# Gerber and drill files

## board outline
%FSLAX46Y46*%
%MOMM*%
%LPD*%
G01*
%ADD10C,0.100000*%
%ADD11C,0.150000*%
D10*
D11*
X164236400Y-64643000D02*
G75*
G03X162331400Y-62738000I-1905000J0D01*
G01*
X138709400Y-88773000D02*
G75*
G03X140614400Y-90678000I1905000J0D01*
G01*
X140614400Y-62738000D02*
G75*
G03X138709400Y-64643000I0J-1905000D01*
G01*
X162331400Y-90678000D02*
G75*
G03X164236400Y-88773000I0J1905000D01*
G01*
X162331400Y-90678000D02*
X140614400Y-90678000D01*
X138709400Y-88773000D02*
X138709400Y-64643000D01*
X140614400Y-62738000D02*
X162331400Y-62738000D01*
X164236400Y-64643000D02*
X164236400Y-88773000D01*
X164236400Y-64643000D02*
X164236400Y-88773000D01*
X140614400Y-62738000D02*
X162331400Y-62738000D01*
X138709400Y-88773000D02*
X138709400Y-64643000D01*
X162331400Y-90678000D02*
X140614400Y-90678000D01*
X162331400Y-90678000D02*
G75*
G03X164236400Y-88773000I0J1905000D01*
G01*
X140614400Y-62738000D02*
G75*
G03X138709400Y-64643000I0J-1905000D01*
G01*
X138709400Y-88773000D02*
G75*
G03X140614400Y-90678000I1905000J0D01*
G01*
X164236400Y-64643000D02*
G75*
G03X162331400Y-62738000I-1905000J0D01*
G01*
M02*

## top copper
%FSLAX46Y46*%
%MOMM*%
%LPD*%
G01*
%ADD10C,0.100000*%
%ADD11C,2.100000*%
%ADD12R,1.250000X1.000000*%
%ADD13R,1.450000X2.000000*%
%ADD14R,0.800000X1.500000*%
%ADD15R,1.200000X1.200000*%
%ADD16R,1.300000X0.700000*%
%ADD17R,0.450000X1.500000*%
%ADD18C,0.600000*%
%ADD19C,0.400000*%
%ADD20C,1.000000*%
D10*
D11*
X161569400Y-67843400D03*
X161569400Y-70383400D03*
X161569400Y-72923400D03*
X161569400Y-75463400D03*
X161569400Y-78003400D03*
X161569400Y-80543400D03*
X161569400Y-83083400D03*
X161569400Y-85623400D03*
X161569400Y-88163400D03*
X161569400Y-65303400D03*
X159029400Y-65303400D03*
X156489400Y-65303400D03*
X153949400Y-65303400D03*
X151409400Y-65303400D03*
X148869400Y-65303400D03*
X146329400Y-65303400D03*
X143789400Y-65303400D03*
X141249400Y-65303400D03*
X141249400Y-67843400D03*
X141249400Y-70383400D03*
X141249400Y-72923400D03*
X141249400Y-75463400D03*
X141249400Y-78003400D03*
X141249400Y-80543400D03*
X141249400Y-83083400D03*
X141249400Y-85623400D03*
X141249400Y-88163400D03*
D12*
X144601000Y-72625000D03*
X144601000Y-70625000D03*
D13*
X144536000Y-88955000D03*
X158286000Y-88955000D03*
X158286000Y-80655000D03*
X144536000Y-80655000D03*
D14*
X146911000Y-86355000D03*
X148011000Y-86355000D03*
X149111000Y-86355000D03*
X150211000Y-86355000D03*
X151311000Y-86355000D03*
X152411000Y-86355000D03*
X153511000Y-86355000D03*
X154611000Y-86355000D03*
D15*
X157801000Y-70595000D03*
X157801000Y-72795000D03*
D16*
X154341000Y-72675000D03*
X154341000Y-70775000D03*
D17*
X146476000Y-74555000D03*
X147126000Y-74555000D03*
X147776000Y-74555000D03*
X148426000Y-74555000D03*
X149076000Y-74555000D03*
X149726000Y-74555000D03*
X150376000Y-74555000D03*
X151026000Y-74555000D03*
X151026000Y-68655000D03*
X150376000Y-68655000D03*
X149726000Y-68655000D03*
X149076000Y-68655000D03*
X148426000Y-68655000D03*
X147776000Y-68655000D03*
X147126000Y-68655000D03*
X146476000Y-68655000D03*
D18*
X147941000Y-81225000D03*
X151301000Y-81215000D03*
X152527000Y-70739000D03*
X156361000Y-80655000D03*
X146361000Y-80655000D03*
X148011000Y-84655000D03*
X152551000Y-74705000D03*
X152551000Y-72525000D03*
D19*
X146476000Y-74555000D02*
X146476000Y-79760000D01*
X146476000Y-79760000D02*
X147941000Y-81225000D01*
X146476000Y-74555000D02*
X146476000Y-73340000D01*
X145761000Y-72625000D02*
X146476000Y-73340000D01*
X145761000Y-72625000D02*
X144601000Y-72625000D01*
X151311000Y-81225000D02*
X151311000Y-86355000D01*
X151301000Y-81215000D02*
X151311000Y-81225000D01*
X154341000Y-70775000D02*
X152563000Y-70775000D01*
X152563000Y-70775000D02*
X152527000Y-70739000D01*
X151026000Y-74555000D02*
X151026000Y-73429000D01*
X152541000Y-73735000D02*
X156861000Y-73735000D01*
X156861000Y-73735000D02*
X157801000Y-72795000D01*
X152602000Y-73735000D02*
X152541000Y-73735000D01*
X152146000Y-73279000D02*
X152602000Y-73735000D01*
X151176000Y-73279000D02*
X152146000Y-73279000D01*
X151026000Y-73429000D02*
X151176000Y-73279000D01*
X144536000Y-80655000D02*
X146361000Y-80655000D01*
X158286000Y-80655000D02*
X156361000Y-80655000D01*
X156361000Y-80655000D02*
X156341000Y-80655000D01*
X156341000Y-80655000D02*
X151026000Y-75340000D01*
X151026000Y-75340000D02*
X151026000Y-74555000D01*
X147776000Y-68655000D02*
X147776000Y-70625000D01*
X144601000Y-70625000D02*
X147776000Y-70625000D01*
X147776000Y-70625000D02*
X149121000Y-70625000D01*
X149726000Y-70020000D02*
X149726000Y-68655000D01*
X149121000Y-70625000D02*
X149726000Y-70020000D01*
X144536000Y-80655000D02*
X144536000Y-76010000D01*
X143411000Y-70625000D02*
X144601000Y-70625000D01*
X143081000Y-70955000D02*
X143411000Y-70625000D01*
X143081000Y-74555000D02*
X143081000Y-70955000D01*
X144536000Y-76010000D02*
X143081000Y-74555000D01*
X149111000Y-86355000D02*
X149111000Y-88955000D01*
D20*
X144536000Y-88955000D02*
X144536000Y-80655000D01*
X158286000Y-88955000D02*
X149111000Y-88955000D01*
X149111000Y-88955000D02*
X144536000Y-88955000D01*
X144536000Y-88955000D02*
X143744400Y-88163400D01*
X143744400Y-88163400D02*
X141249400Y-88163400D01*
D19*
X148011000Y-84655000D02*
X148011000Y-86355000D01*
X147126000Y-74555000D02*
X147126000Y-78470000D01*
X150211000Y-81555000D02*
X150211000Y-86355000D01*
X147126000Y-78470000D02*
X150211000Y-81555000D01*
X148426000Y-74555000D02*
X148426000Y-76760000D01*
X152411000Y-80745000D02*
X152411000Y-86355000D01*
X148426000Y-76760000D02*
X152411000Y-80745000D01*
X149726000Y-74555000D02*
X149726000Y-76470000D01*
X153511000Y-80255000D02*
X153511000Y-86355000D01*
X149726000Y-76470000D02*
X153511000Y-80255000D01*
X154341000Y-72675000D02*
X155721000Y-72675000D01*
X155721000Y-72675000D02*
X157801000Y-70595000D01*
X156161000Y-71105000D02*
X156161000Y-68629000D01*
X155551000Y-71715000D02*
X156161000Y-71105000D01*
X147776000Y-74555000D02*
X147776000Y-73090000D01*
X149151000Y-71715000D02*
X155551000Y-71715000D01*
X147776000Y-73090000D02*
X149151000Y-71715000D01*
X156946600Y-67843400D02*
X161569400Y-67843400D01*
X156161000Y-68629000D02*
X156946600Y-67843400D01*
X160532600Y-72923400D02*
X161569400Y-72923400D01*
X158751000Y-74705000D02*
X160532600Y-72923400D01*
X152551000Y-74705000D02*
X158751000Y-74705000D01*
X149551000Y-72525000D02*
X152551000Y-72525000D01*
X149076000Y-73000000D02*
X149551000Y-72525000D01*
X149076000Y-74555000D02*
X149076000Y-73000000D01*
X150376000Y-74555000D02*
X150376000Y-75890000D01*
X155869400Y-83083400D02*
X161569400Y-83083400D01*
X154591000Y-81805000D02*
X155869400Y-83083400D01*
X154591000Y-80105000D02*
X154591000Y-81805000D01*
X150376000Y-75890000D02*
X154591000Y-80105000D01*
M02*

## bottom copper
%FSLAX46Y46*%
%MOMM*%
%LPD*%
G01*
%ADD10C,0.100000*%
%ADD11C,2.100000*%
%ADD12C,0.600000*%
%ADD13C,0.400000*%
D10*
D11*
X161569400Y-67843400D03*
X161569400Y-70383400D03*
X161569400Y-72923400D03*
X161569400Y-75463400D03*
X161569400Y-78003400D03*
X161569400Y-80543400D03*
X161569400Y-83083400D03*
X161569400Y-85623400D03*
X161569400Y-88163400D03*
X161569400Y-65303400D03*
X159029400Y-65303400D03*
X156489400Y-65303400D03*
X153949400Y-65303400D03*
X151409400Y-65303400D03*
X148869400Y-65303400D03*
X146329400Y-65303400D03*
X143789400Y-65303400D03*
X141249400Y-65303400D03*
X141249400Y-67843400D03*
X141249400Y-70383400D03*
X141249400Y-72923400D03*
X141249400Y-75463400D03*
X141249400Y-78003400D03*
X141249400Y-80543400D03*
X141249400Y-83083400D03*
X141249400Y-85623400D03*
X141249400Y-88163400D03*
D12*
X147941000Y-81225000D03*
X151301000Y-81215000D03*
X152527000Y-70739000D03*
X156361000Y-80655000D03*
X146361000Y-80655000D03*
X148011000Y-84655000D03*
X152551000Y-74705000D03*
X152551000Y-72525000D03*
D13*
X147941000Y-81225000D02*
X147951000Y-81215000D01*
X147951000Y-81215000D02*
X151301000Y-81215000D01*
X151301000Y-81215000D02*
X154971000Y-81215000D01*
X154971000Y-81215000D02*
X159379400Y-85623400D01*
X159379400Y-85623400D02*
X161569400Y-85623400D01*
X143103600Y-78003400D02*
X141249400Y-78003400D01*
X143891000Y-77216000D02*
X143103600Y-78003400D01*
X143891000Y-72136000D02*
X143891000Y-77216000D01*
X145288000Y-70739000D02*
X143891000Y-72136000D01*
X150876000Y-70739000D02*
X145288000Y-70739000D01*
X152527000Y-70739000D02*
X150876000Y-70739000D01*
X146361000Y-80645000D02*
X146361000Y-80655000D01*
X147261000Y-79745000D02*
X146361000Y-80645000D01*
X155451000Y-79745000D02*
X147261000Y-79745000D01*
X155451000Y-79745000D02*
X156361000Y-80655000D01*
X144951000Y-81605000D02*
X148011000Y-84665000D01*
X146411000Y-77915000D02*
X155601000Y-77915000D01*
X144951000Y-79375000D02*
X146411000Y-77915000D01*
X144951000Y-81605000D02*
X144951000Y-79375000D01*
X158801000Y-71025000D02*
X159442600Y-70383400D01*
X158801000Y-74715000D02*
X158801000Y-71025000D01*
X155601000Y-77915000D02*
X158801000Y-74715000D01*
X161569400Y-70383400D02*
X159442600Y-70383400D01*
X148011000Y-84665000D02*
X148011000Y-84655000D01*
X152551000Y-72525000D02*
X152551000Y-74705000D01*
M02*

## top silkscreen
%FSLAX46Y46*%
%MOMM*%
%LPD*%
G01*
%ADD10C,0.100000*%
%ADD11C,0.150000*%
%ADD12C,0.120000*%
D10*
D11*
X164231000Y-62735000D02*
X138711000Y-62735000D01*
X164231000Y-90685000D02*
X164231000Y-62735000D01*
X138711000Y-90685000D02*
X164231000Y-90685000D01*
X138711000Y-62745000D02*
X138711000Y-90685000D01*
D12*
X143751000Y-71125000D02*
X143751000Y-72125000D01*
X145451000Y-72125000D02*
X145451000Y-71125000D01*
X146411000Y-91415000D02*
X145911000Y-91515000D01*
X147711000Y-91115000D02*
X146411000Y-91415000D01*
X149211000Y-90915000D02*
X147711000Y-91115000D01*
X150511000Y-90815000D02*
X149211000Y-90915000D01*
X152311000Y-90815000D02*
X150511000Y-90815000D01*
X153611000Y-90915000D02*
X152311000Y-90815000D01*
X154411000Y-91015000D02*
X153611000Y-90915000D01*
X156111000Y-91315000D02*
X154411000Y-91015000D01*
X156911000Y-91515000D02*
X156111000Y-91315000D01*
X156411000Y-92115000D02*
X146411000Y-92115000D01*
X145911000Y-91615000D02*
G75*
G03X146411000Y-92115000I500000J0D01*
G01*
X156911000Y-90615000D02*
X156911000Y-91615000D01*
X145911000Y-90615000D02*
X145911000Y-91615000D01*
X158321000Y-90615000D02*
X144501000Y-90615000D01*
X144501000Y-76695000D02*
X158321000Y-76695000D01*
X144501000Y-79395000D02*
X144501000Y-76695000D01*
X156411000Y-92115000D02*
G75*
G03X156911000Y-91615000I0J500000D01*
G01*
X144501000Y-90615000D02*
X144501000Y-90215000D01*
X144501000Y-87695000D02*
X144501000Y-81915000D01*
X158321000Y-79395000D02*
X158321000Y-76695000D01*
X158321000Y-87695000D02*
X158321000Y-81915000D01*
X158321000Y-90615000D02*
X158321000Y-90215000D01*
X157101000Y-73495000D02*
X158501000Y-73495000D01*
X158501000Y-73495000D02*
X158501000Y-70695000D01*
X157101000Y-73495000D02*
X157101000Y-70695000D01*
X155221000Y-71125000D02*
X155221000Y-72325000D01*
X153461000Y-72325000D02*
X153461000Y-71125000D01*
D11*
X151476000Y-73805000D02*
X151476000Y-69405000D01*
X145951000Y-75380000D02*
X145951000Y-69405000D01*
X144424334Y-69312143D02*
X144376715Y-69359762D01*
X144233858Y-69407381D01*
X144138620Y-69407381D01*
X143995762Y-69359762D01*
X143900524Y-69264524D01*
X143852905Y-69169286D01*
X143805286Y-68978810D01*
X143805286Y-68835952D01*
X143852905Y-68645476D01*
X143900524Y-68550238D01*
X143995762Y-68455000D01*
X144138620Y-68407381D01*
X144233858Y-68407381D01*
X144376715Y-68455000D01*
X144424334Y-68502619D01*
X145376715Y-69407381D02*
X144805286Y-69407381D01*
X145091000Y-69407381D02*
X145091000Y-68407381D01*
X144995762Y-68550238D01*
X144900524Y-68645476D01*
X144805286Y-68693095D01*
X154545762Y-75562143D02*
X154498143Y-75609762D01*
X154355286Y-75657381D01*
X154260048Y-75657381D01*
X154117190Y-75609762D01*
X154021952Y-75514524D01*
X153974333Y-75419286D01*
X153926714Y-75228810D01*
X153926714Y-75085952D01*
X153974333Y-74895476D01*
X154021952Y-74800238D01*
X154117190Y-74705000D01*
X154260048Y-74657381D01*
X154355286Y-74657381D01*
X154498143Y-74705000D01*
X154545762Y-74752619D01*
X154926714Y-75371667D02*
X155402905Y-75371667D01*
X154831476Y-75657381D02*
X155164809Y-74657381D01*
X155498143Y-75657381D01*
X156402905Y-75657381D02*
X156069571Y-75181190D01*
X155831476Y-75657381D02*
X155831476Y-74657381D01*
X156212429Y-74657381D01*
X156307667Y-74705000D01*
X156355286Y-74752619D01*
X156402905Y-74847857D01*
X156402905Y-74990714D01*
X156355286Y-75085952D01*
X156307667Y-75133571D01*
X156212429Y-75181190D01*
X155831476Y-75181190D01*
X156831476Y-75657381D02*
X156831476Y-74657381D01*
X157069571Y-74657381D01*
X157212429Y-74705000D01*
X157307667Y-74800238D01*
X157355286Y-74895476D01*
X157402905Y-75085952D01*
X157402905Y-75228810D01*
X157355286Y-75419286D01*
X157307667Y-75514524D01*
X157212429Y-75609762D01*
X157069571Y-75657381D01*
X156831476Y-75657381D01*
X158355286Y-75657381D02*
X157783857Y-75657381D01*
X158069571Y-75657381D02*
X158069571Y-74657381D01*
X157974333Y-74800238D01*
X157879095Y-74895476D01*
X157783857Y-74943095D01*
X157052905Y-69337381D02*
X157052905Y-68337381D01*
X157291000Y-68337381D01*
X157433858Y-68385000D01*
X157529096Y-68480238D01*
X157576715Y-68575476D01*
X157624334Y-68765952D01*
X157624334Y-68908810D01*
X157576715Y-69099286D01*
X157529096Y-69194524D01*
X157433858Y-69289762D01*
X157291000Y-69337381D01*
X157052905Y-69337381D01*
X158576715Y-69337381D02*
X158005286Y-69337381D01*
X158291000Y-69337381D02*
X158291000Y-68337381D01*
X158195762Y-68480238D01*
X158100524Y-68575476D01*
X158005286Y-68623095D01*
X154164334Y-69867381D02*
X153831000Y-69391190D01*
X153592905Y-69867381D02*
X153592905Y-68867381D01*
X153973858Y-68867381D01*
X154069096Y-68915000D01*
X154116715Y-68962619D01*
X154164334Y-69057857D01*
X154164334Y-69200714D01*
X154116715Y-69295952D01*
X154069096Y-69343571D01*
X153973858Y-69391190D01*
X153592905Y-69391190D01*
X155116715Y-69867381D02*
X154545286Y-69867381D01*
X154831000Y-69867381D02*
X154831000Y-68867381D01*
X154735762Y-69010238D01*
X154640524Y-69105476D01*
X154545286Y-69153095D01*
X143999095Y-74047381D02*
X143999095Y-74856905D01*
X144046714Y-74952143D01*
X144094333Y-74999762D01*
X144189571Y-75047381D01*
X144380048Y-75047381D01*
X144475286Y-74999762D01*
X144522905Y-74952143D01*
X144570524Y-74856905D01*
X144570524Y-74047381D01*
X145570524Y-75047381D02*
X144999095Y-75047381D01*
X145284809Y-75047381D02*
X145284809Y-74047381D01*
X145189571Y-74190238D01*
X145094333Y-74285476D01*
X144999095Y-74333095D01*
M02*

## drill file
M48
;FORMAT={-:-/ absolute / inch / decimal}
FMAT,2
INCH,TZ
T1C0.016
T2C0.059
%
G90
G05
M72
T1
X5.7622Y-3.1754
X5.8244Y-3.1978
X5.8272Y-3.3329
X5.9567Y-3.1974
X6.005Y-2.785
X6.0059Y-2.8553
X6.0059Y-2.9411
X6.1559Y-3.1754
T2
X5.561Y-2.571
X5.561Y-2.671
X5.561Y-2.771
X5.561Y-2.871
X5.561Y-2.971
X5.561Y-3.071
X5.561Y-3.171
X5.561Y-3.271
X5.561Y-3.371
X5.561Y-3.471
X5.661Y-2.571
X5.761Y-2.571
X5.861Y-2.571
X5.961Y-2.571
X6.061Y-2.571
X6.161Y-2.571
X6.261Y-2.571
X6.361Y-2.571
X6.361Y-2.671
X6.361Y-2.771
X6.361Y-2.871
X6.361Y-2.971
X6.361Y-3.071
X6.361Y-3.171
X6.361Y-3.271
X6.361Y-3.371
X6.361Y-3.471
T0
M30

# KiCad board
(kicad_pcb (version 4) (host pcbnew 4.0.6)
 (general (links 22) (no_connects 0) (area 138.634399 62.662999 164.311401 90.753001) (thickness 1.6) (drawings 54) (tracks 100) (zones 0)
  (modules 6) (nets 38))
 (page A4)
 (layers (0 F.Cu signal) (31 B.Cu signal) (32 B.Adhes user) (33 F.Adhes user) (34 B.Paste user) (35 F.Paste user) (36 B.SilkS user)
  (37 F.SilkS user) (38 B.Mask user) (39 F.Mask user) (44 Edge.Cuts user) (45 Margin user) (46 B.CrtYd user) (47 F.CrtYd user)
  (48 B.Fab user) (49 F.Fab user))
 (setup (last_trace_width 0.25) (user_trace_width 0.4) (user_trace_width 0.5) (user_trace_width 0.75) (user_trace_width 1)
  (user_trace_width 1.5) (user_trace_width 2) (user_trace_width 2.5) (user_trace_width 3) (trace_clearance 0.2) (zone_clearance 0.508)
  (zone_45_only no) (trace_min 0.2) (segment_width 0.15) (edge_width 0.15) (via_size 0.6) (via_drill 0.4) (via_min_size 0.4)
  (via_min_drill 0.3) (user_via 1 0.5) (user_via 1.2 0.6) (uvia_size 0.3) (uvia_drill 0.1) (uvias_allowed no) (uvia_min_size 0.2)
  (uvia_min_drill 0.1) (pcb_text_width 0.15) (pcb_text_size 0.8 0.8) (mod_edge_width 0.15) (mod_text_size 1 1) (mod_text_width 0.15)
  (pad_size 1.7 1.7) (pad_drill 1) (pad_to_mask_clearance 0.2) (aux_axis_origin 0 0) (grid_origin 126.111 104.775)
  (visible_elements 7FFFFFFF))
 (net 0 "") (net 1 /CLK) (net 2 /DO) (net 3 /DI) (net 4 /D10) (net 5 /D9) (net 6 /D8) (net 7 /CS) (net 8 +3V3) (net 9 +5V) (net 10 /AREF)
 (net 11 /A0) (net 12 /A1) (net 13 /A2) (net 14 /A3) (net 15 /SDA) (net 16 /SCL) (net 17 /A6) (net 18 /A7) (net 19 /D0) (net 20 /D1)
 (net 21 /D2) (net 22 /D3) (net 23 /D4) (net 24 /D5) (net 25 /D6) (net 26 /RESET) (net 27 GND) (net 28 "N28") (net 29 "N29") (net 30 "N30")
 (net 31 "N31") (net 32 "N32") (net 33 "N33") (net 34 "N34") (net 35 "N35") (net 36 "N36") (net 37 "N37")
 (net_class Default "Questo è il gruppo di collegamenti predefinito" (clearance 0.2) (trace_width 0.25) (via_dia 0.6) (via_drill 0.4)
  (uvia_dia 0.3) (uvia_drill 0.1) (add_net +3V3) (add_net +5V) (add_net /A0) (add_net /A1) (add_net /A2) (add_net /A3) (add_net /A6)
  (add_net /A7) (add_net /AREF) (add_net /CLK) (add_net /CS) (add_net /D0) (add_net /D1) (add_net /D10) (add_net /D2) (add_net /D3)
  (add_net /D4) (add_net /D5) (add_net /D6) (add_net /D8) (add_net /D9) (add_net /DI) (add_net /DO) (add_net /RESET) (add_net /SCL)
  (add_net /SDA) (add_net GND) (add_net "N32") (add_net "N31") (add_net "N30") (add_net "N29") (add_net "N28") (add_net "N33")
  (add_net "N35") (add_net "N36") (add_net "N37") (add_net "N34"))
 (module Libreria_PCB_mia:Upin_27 (layer B.Cu) (at 161.5694 88.1634 180)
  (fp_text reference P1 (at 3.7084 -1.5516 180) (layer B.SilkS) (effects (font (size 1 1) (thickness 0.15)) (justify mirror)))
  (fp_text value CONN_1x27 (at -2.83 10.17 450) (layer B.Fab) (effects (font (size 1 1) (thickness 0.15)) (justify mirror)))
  (pad 9 thru_hole circle (at 0 20.32 180) (size 2.1 2.1) (drill 1.5) (layers *.Cu *.Mask) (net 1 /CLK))
  (pad 8 thru_hole circle (at 0 17.78 180) (size 2.1 2.1) (drill 1.5) (layers *.Cu *.Mask) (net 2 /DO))
  (pad 7 thru_hole circle (at 0 15.24 180) (size 2.1 2.1) (drill 1.5) (layers *.Cu *.Mask) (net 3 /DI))
  (pad 6 thru_hole circle (at 0 12.7 180) (size 2.1 2.1) (drill 1.5) (layers *.Cu *.Mask) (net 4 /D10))
  (pad 5 thru_hole circle (at 0 10.16 180) (size 2.1 2.1) (drill 1.5) (layers *.Cu *.Mask) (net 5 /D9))
  (pad 4 thru_hole circle (at 0 7.62 180) (size 2.1 2.1) (drill 1.5) (layers *.Cu *.Mask) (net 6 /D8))
  (pad 3 thru_hole circle (at 0 5.08 180) (size 2.1 2.1) (drill 1.5) (layers *.Cu *.Mask) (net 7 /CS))
  (pad 2 thru_hole circle (at 0 2.54 180) (size 2.1 2.1) (drill 1.5) (layers *.Cu *.Mask) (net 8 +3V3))
  (pad 1 thru_hole circle (at 0 0 180) (size 2.1 2.1) (drill 1.5) (layers *.Cu *.Mask) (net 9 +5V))
  (pad 10 thru_hole circle (at 0 22.86 180) (size 2.1 2.1) (drill 1.5) (layers *.Cu *.Mask) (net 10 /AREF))
  (pad 11 thru_hole circle (at 2.54 22.86 180) (size 2.1 2.1) (drill 1.5) (layers *.Cu *.Mask) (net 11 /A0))
  (pad 12 thru_hole circle (at 5.08 22.86 180) (size 2.1 2.1) (drill 1.5) (layers *.Cu *.Mask) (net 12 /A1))
  (pad 13 thru_hole circle (at 7.62 22.86 180) (size 2.1 2.1) (drill 1.5) (layers *.Cu *.Mask) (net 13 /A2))
  (pad 14 thru_hole circle (at 10.16 22.86 180) (size 2.1 2.1) (drill 1.5) (layers *.Cu *.Mask) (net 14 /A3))
  (pad 15 thru_hole circle (at 12.7 22.86 180) (size 2.1 2.1) (drill 1.5) (layers *.Cu *.Mask) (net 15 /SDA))
  (pad 16 thru_hole circle (at 15.24 22.86 180) (size 2.1 2.1) (drill 1.5) (layers *.Cu *.Mask) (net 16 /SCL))
  (pad 17 thru_hole circle (at 17.78 22.86 180) (size 2.1 2.1) (drill 1.5) (layers *.Cu *.Mask) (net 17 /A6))
  (pad 18 thru_hole circle (at 20.32 22.86 180) (size 2.1 2.1) (drill 1.5) (layers *.Cu *.Mask) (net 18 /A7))
  (pad 19 thru_hole circle (at 20.32 20.32 180) (size 2.1 2.1) (drill 1.5) (layers *.Cu *.Mask) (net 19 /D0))
  (pad 20 thru_hole circle (at 20.32 17.78 180) (size 2.1 2.1) (drill 1.5) (layers *.Cu *.Mask) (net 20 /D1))
  (pad 21 thru_hole circle (at 20.32 15.24 180) (size 2.1 2.1) (drill 1.5) (layers *.Cu *.Mask) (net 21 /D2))
  (pad 22 thru_hole circle (at 20.32 12.7 180) (size 2.1 2.1) (drill 1.5) (layers *.Cu *.Mask) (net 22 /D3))
  (pad 23 thru_hole circle (at 20.32 10.16 180) (size 2.1 2.1) (drill 1.5) (layers *.Cu *.Mask) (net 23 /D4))
  (pad 24 thru_hole circle (at 20.32 7.62 180) (size 2.1 2.1) (drill 1.5) (layers *.Cu *.Mask) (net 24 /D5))
  (pad 25 thru_hole circle (at 20.32 5.08 180) (size 2.1 2.1) (drill 1.5) (layers *.Cu *.Mask) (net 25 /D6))
  (pad 26 thru_hole circle (at 20.32 2.54 180) (size 2.1 2.1) (drill 1.5) (layers *.Cu *.Mask) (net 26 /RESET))
  (pad 27 thru_hole circle (at 20.32 0 180) (size 2.1 2.1) (drill 1.5) (layers *.Cu *.Mask) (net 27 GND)))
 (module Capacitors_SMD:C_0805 (layer F.Cu) (at 144.601 71.625 90)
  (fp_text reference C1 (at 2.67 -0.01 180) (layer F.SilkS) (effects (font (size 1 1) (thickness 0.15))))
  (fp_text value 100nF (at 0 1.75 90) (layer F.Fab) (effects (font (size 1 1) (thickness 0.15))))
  (fp_line (start 0.5 -0.85) (end -0.5 -0.85) (layer F.SilkS) (width 0.12))
  (fp_line (start -0.5 0.85) (end 0.5 0.85) (layer F.SilkS) (width 0.12))
  (pad 1 smd rect (at -1 0 90) (size 1 1.25) (layers F.Cu F.Paste F.Mask) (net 8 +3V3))
  (pad 2 smd rect (at 1 0 90) (size 1 1.25) (layers F.Cu F.Paste F.Mask) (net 27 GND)))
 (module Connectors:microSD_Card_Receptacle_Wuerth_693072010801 (layer F.Cu) (at 151.411 83.655 180)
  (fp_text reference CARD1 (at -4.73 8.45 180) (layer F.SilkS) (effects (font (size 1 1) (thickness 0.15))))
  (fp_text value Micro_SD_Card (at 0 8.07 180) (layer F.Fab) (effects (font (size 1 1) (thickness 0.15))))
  (fp_line (start 5 -7.76) (end 5.5 -7.86) (layer F.SilkS) (width 0.12))
  (fp_line (start 3.7 -7.46) (end 5 -7.76) (layer F.SilkS) (width 0.12))
  (fp_line (start 2.2 -7.26) (end 3.7 -7.46) (layer F.SilkS) (width 0.12))
  (fp_line (start 0.9 -7.16) (end 2.2 -7.26) (layer F.SilkS) (width 0.12))
  (fp_line (start -0.9 -7.16) (end 0.9 -7.16) (layer F.SilkS) (width 0.12))
  (fp_line (start -2.2 -7.26) (end -0.9 -7.16) (layer F.SilkS) (width 0.12))
  (fp_line (start -3 -7.36) (end -2.2 -7.26) (layer F.SilkS) (width 0.12))
  (fp_line (start -4.7 -7.66) (end -3 -7.36) (layer F.SilkS) (width 0.12))
  (fp_line (start -5.5 -7.86) (end -4.7 -7.66) (layer F.SilkS) (width 0.12))
  (fp_line (start -5 -8.46) (end 5 -8.46) (layer F.SilkS) (width 0.12))
  (fp_arc (start 5 -7.96) (end 5 -8.46) (angle 90) (layer F.SilkS) (width 0.12))
  (fp_line (start -5.5 -6.96) (end -5.5 -7.96) (layer F.SilkS) (width 0.12))
  (fp_line (start 5.5 -6.96) (end 5.5 -7.96) (layer F.SilkS) (width 0.12))
  (fp_line (start -6.91 -6.96) (end 6.91 -6.96) (layer F.SilkS) (width 0.12))
  (fp_line (start 6.91 6.96) (end -6.91 6.96) (layer F.SilkS) (width 0.12))
  (fp_line (start 6.91 4.26) (end 6.91 6.96) (layer F.SilkS) (width 0.12))
  (fp_arc (start -5 -7.96) (end -5.5 -7.96) (angle 90) (layer F.SilkS) (width 0.12))
  (fp_line (start 6.91 -6.96) (end 6.91 -6.56) (layer F.SilkS) (width 0.12))
  (fp_line (start 6.91 -4.04) (end 6.91 1.74) (layer F.SilkS) (width 0.12))
  (fp_line (start -6.91 4.26) (end -6.91 6.96) (layer F.SilkS) (width 0.12))
  (fp_line (start -6.91 -4.04) (end -6.91 1.74) (layer F.SilkS) (width 0.12))
  (fp_line (start -6.91 -6.96) (end -6.91 -6.56) (layer F.SilkS) (width 0.12))
  (pad 9 smd rect (at 6.875 -5.3 180) (size 1.45 2) (layers F.Cu F.Paste F.Mask) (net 27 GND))
  (pad 9 smd rect (at -6.875 -5.3 180) (size 1.45 2) (layers F.Cu F.Paste F.Mask) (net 27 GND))
  (pad 9 smd rect (at -6.875 3 180) (size 1.45 2) (layers F.Cu F.Paste F.Mask) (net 27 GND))
  (pad 9 smd rect (at 6.875 3 180) (size 1.45 2) (layers F.Cu F.Paste F.Mask) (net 27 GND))
  (pad 8 smd rect (at 4.5 -2.7 180) (size 0.8 1.5) (layers F.Cu F.Paste F.Mask) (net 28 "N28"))
  (pad 7 smd rect (at 3.4 -2.7 180) (size 0.8 1.5) (layers F.Cu F.Paste F.Mask) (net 2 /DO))
  (pad 6 smd rect (at 2.3 -2.7 180) (size 0.8 1.5) (layers F.Cu F.Paste F.Mask) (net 27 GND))
  (pad 5 smd rect (at 1.2 -2.7 180) (size 0.8 1.5) (layers F.Cu F.Paste F.Mask) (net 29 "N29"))
  (pad 4 smd rect (at 0.1 -2.7 180) (size 0.8 1.5) (layers F.Cu F.Paste F.Mask) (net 8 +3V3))
  (pad 3 smd rect (at -1 -2.7 180) (size 0.8 1.5) (layers F.Cu F.Paste F.Mask) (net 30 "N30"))
  (pad 2 smd rect (at -2.1 -2.7 180) (size 0.8 1.5) (layers F.Cu F.Paste F.Mask) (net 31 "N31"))
  (pad 1 smd rect (at -3.2 -2.7 180) (size 0.8 1.5) (layers F.Cu F.Paste F.Mask) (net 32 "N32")))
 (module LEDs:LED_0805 (layer F.Cu) (at 157.801 71.695 90)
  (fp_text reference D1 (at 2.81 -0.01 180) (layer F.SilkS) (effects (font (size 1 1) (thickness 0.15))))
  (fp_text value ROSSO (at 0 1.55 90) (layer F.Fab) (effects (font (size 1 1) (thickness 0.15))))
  (fp_line (start -1.8 -0.7) (end -1.8 0.7) (layer F.SilkS) (width 0.12))
  (fp_line (start -1.8 0.7) (end 1 0.7) (layer F.SilkS) (width 0.12))
  (fp_line (start -1.8 -0.7) (end 1 -0.7) (layer F.SilkS) (width 0.12))
  (pad 2 smd rect (at 1.1 0 270) (size 1.2 1.2) (layers F.Cu F.Paste F.Mask) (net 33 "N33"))
  (pad 1 smd rect (at -1.1 0 270) (size 1.2 1.2) (layers F.Cu F.Paste F.Mask) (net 27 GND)))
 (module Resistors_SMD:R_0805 (layer F.Cu) (at 154.341 71.725 90)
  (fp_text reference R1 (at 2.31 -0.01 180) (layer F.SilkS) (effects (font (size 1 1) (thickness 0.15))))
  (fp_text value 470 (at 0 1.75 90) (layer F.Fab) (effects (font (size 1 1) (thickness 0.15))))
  (fp_line (start 0.6 0.88) (end -0.6 0.88) (layer F.SilkS) (width 0.12))
  (fp_line (start -0.6 -0.88) (end 0.6 -0.88) (layer F.SilkS) (width 0.12))
  (pad 1 smd rect (at -0.95 0 90) (size 0.7 1.3) (layers F.Cu F.Paste F.Mask) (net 33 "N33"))
  (pad 2 smd rect (at 0.95 0 90) (size 0.7 1.3) (layers F.Cu F.Paste F.Mask) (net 23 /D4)))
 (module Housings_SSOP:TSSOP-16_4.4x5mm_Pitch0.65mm (layer F.Cu) (at 148.751 71.605 90)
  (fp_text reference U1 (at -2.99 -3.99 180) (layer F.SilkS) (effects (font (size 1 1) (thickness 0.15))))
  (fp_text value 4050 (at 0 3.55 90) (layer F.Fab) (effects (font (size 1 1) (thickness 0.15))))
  (fp_line (start -2.2 2.725) (end 2.2 2.725) (layer F.SilkS) (width 0.15))
  (fp_line (start -3.775 -2.8) (end 2.2 -2.8) (layer F.SilkS) (width 0.15))
  (pad 1 smd rect (at -2.95 -2.275 90) (size 1.5 0.45) (layers F.Cu F.Paste F.Mask) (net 8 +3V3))
  (pad 2 smd rect (at -2.95 -1.625 90) (size 1.5 0.45) (layers F.Cu F.Paste F.Mask) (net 29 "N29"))
  (pad 3 smd rect (at -2.95 -0.975 90) (size 1.5 0.45) (layers F.Cu F.Paste F.Mask) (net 1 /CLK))
  (pad 4 smd rect (at -2.95 -0.325 90) (size 1.5 0.45) (layers F.Cu F.Paste F.Mask) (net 30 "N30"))
  (pad 5 smd rect (at -2.95 0.325 90) (size 1.5 0.45) (layers F.Cu F.Paste F.Mask) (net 3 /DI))
  (pad 6 smd rect (at -2.95 0.975 90) (size 1.5 0.45) (layers F.Cu F.Paste F.Mask) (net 31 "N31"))
  (pad 7 smd rect (at -2.95 1.625 90) (size 1.5 0.45) (layers F.Cu F.Paste F.Mask) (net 7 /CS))
  (pad 8 smd rect (at -2.95 2.275 90) (size 1.5 0.45) (layers F.Cu F.Paste F.Mask) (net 27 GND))
  (pad 9 smd rect (at 2.95 2.275 90) (size 1.5 0.45) (layers F.Cu F.Paste F.Mask) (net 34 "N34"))
  (pad 10 smd rect (at 2.95 1.625 90) (size 1.5 0.45) (layers F.Cu F.Paste F.Mask) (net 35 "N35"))
  (pad 11 smd rect (at 2.95 0.975 90) (size 1.5 0.45) (layers F.Cu F.Paste F.Mask) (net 27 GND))
  (pad 12 smd rect (at 2.95 0.325 90) (size 1.5 0.45) (layers F.Cu F.Paste F.Mask) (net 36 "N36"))
  (pad 13 smd rect (at 2.95 -0.325 90) (size 1.5 0.45) (layers F.Cu F.Paste F.Mask))
  (pad 14 smd rect (at 2.95 -0.975 90) (size 1.5 0.45) (layers F.Cu F.Paste F.Mask) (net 27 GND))
  (pad 15 smd rect (at 2.95 -1.625 90) (size 1.5 0.45) (layers F.Cu F.Paste F.Mask) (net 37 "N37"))
  (pad 16 smd rect (at 2.95 -2.275 90) (size 1.5 0.45) (layers F.Cu F.Paste F.Mask)))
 (gr_line (start 164.231 62.735) (end 138.711 62.735) (angle 90) (layer F.SilkS) (width 0.15))
 (gr_line (start 164.231 90.685) (end 164.231 62.735) (angle 90) (layer F.SilkS) (width 0.15))
 (gr_line (start 138.711 90.685) (end 164.231 90.685) (angle 90) (layer F.SilkS) (width 0.15))
 (gr_line (start 138.711 62.745) (end 138.711 90.685) (angle 90) (layer F.SilkS) (width 0.15))
 (gr_arc (start 162.3314 64.643) (end 162.3314 62.738) (angle 90) (layer Edge.Cuts) (width 0.15))
 (gr_arc (start 140.6144 88.773) (end 140.6144 90.678) (angle 90) (layer Edge.Cuts) (width 0.15))
 (gr_arc (start 140.6144 64.643) (end 138.7094 64.643) (angle 90) (layer Edge.Cuts) (width 0.15))
 (gr_arc (start 162.3314 88.773) (end 164.2364 88.773) (angle 90) (layer Edge.Cuts) (width 0.15))
 (gr_line (start 162.3314 90.678) (end 140.6144 90.678) (angle 90) (layer Edge.Cuts) (width 0.15))
 (gr_line (start 138.7094 88.773) (end 138.7094 64.643) (angle 90) (layer Edge.Cuts) (width 0.15))
 (gr_line (start 140.6144 62.738) (end 162.3314 62.738) (angle 90) (layer Edge.Cuts) (width 0.15))
 (gr_line (start 164.2364 64.643) (end 164.2364 88.773) (angle 90) (layer Edge.Cuts) (width 0.15))
 (gr_line (start 164.2364 64.643) (end 164.2364 88.773) (angle 90) (layer Edge.Cuts) (width 0.15))
 (gr_line (start 140.6144 62.738) (end 162.3314 62.738) (angle 90) (layer Edge.Cuts) (width 0.15))
 (gr_line (start 138.7094 88.773) (end 138.7094 64.643) (angle 90) (layer Edge.Cuts) (width 0.15))
 (gr_line (start 162.3314 90.678) (end 140.6144 90.678) (angle 90) (layer Edge.Cuts) (width 0.15))
 (gr_arc (start 162.3314 88.773) (end 164.2364 88.773) (angle 90) (layer Edge.Cuts) (width 0.15))
 (gr_arc (start 140.6144 64.643) (end 138.7094 64.643) (angle 90) (layer Edge.Cuts) (width 0.15))
 (gr_arc (start 140.6144 88.773) (end 140.6144 90.678) (angle 90) (layer Edge.Cuts) (width 0.15))
 (gr_arc (start 162.3314 64.643) (end 162.3314 62.738) (angle 90) (layer Edge.Cuts) (width 0.15))
 (segment (start 146.476 74.555) (end 146.476 79.76) (width 0.4) (layer F.Cu) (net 8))
 (segment (start 146.476 79.76) (end 147.941 81.225) (width 0.4) (layer F.Cu) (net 8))
 (via (at 147.941 81.225) (size 0.6) (drill 0.4) (layers F.Cu B.Cu) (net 8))
 (segment (start 147.941 81.225) (end 147.951 81.215) (width 0.4) (layer B.Cu) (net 8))
 (segment (start 147.951 81.215) (end 151.301 81.215) (width 0.4) (layer B.Cu) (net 8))
 (segment (start 146.476 74.555) (end 146.476 73.34) (width 0.4) (layer F.Cu) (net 8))
 (segment (start 145.761 72.625) (end 146.476 73.34) (width 0.4) (layer F.Cu) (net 8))
 (segment (start 145.761 72.625) (end 144.601 72.625) (width 0.4) (layer F.Cu) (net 8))
 (segment (start 151.301 81.215) (end 154.971 81.215) (width 0.4) (layer B.Cu) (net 8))
 (segment (start 154.971 81.215) (end 159.3794 85.6234) (width 0.4) (layer B.Cu) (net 8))
 (segment (start 159.3794 85.6234) (end 161.5694 85.6234) (width 0.4) (layer B.Cu) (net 8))
 (segment (start 151.311 81.225) (end 151.311 86.355) (width 0.4) (layer F.Cu) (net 8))
 (via (at 151.301 81.215) (size 0.6) (drill 0.4) (layers F.Cu B.Cu) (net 8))
 (segment (start 151.301 81.215) (end 151.311 81.225) (width 0.4) (layer F.Cu) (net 8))
 (segment (start 154.341 70.775) (end 152.563 70.775) (width 0.4) (layer F.Cu) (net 23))
 (segment (start 143.1036 78.0034) (end 141.2494 78.0034) (width 0.4) (layer B.Cu) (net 23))
 (segment (start 143.891 77.216) (end 143.1036 78.0034) (width 0.4) (layer B.Cu) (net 23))
 (segment (start 143.891 72.136) (end 143.891 77.216) (width 0.4) (layer B.Cu) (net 23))
 (segment (start 145.288 70.739) (end 143.891 72.136) (width 0.4) (layer B.Cu) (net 23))
 (segment (start 150.876 70.739) (end 145.288 70.739) (width 0.4) (layer B.Cu) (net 23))
 (segment (start 152.527 70.739) (end 150.876 70.739) (width 0.4) (layer B.Cu) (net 23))
 (via (at 152.527 70.739) (size 0.6) (drill 0.4) (layers F.Cu B.Cu) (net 23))
 (segment (start 152.563 70.775) (end 152.527 70.739) (width 0.4) (layer F.Cu) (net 23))
 (segment (start 151.026 74.555) (end 151.026 73.429) (width 0.4) (layer F.Cu) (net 27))
 (segment (start 152.541 73.735) (end 156.861 73.735) (width 0.4) (layer F.Cu) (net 27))
 (segment (start 156.861 73.735) (end 157.801 72.795) (width 0.4) (layer F.Cu) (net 27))
 (segment (start 152.602 73.735) (end 152.541 73.735) (width 0.4) (layer F.Cu) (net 27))
 (segment (start 152.146 73.279) (end 152.602 73.735) (width 0.4) (layer F.Cu) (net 27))
 (segment (start 151.176 73.279) (end 152.146 73.279) (width 0.4) (layer F.Cu) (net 27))
 (segment (start 151.026 73.429) (end 151.176 73.279) (width 0.4) (layer F.Cu) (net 27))
 (via (at 156.361 80.655) (size 0.6) (drill 0.4) (layers F.Cu B.Cu) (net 27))
 (segment (start 144.536 80.655) (end 146.361 80.655) (width 0.4) (layer F.Cu) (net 27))
 (via (at 146.361 80.655) (size 0.6) (drill 0.4) (layers F.Cu B.Cu) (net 27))
 (segment (start 146.361 80.645) (end 146.361 80.655) (width 0.4) (layer B.Cu) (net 27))
 (segment (start 147.261 79.745) (end 146.361 80.645) (width 0.4) (layer B.Cu) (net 27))
 (segment (start 155.451 79.745) (end 147.261 79.745) (width 0.4) (layer B.Cu) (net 27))
 (segment (start 155.451 79.745) (end 156.361 80.655) (width 0.4) (layer B.Cu) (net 27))
 (segment (start 158.286 80.655) (end 156.361 80.655) (width 0.4) (layer F.Cu) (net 27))
 (segment (start 156.361 80.655) (end 156.341 80.655) (width 0.4) (layer F.Cu) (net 27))
 (segment (start 156.341 80.655) (end 151.026 75.34) (width 0.4) (layer F.Cu) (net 27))
 (segment (start 151.026 75.34) (end 151.026 74.555) (width 0.4) (layer F.Cu) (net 27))
 (segment (start 147.776 68.655) (end 147.776 70.625) (width 0.4) (layer F.Cu) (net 27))
 (segment (start 144.601 70.625) (end 147.776 70.625) (width 0.4) (layer F.Cu) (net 27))
 (segment (start 147.776 70.625) (end 149.121 70.625) (width 0.4) (layer F.Cu) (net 27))
 (segment (start 149.726 70.02) (end 149.726 68.655) (width 0.4) (layer F.Cu) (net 27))
 (segment (start 149.121 70.625) (end 149.726 70.02) (width 0.4) (layer F.Cu) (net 27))
 (segment (start 144.536 80.655) (end 144.536 76.01) (width 0.4) (layer F.Cu) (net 27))
 (segment (start 143.411 70.625) (end 144.601 70.625) (width 0.4) (layer F.Cu) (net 27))
 (segment (start 143.081 70.955) (end 143.411 70.625) (width 0.4) (layer F.Cu) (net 27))
 (segment (start 143.081 74.555) (end 143.081 70.955) (width 0.4) (layer F.Cu) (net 27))
 (segment (start 144.536 76.01) (end 143.081 74.555) (width 0.4) (layer F.Cu) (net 27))
 (segment (start 149.111 86.355) (end 149.111 88.955) (width 0.4) (layer F.Cu) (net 27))
 (segment (start 144.536 88.955) (end 144.536 80.655) (width 1) (layer F.Cu) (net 27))
 (segment (start 158.286 88.955) (end 149.111 88.955) (width 1) (layer F.Cu) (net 27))
 (segment (start 149.111 88.955) (end 144.536 88.955) (width 1) (layer F.Cu) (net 27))
 (segment (start 144.536 88.955) (end 143.7444 88.1634) (width 1) (layer F.Cu) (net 27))
 (segment (start 143.7444 88.1634) (end 141.2494 88.1634) (width 1) (layer F.Cu) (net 27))
 (segment (start 144.951 81.605) (end 148.011 84.665) (width 0.4) (layer B.Cu) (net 2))
 (segment (start 146.411 77.915) (end 155.601 77.915) (width 0.4) (layer B.Cu) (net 2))
 (segment (start 144.951 79.375) (end 146.411 77.915) (width 0.4) (layer B.Cu) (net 2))
 (segment (start 144.951 81.605) (end 144.951 79.375) (width 0.4) (layer B.Cu) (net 2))
 (segment (start 158.801 71.025) (end 159.4426 70.3834) (width 0.4) (layer B.Cu) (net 2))
 (segment (start 158.801 74.715) (end 158.801 71.025) (width 0.4) (layer B.Cu) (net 2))
 (segment (start 155.601 77.915) (end 158.801 74.715) (width 0.4) (layer B.Cu) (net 2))
 (segment (start 161.5694 70.3834) (end 159.4426 70.3834) (width 0.4) (layer B.Cu) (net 2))
 (segment (start 148.011 84.655) (end 148.011 86.355) (width 0.4) (layer F.Cu) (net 2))
 (via (at 148.011 84.655) (size 0.6) (drill 0.4) (layers F.Cu B.Cu) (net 2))
 (segment (start 148.011 84.665) (end 148.011 84.655) (width 0.4) (layer B.Cu) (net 2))
 (segment (start 147.126 74.555) (end 147.126 78.47) (width 0.4) (layer F.Cu) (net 29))
 (segment (start 150.211 81.555) (end 150.211 86.355) (width 0.4) (layer F.Cu) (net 29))
 (segment (start 147.126 78.47) (end 150.211 81.555) (width 0.4) (layer F.Cu) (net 29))
 (segment (start 148.426 74.555) (end 148.426 76.76) (width 0.4) (layer F.Cu) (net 30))
 (segment (start 152.411 80.745) (end 152.411 86.355) (width 0.4) (layer F.Cu) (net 30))
 (segment (start 148.426 76.76) (end 152.411 80.745) (width 0.4) (layer F.Cu) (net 30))
 (segment (start 149.726 74.555) (end 149.726 76.47) (width 0.4) (layer F.Cu) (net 31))
 (segment (start 153.511 80.255) (end 153.511 86.355) (width 0.4) (layer F.Cu) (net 31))
 (segment (start 149.726 76.47) (end 153.511 80.255) (width 0.4) (layer F.Cu) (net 31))
 (segment (start 154.341 72.675) (end 155.721 72.675) (width 0.4) (layer F.Cu) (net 33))
 (segment (start 155.721 72.675) (end 157.801 70.595) (width 0.4) (layer F.Cu) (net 33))
 (segment (start 156.161 71.105) (end 156.161 68.629) (width 0.4) (layer F.Cu) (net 1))
 (segment (start 155.551 71.715) (end 156.161 71.105) (width 0.4) (layer F.Cu) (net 1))
 (segment (start 147.776 74.555) (end 147.776 73.09) (width 0.4) (layer F.Cu) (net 1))
 (segment (start 149.151 71.715) (end 155.551 71.715) (width 0.4) (layer F.Cu) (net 1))
 (segment (start 147.776 73.09) (end 149.151 71.715) (width 0.4) (layer F.Cu) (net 1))
 (segment (start 156.9466 67.8434) (end 161.5694 67.8434) (width 0.4) (layer F.Cu) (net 1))
 (segment (start 156.161 68.629) (end 156.9466 67.8434) (width 0.4) (layer F.Cu) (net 1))
 (segment (start 160.5326 72.9234) (end 161.5694 72.9234) (width 0.4) (layer F.Cu) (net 3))
 (segment (start 158.751 74.705) (end 160.5326 72.9234) (width 0.4) (layer F.Cu) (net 3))
 (segment (start 152.551 74.705) (end 158.751 74.705) (width 0.4) (layer F.Cu) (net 3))
 (via (at 152.551 74.705) (size 0.6) (drill 0.4) (layers F.Cu B.Cu) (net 3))
 (segment (start 152.551 72.525) (end 152.551 74.705) (width 0.4) (layer B.Cu) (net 3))
 (via (at 152.551 72.525) (size 0.6) (drill 0.4) (layers F.Cu B.Cu) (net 3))
 (segment (start 149.551 72.525) (end 152.551 72.525) (width 0.4) (layer F.Cu) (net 3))
 (segment (start 149.076 73) (end 149.551 72.525) (width 0.4) (layer F.Cu) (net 3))
 (segment (start 149.076 74.555) (end 149.076 73) (width 0.4) (layer F.Cu) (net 3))
 (segment (start 150.376 74.555) (end 150.376 75.89) (width 0.4) (layer F.Cu) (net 7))
 (segment (start 155.8694 83.0834) (end 161.5694 83.0834) (width 0.4) (layer F.Cu) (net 7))
 (segment (start 154.591 81.805) (end 155.8694 83.0834) (width 0.4) (layer F.Cu) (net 7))
 (segment (start 154.591 80.105) (end 154.591 81.805) (width 0.4) (layer F.Cu) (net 7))
 (segment (start 150.376 75.89) (end 154.591 80.105) (width 0.4) (layer F.Cu) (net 7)))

